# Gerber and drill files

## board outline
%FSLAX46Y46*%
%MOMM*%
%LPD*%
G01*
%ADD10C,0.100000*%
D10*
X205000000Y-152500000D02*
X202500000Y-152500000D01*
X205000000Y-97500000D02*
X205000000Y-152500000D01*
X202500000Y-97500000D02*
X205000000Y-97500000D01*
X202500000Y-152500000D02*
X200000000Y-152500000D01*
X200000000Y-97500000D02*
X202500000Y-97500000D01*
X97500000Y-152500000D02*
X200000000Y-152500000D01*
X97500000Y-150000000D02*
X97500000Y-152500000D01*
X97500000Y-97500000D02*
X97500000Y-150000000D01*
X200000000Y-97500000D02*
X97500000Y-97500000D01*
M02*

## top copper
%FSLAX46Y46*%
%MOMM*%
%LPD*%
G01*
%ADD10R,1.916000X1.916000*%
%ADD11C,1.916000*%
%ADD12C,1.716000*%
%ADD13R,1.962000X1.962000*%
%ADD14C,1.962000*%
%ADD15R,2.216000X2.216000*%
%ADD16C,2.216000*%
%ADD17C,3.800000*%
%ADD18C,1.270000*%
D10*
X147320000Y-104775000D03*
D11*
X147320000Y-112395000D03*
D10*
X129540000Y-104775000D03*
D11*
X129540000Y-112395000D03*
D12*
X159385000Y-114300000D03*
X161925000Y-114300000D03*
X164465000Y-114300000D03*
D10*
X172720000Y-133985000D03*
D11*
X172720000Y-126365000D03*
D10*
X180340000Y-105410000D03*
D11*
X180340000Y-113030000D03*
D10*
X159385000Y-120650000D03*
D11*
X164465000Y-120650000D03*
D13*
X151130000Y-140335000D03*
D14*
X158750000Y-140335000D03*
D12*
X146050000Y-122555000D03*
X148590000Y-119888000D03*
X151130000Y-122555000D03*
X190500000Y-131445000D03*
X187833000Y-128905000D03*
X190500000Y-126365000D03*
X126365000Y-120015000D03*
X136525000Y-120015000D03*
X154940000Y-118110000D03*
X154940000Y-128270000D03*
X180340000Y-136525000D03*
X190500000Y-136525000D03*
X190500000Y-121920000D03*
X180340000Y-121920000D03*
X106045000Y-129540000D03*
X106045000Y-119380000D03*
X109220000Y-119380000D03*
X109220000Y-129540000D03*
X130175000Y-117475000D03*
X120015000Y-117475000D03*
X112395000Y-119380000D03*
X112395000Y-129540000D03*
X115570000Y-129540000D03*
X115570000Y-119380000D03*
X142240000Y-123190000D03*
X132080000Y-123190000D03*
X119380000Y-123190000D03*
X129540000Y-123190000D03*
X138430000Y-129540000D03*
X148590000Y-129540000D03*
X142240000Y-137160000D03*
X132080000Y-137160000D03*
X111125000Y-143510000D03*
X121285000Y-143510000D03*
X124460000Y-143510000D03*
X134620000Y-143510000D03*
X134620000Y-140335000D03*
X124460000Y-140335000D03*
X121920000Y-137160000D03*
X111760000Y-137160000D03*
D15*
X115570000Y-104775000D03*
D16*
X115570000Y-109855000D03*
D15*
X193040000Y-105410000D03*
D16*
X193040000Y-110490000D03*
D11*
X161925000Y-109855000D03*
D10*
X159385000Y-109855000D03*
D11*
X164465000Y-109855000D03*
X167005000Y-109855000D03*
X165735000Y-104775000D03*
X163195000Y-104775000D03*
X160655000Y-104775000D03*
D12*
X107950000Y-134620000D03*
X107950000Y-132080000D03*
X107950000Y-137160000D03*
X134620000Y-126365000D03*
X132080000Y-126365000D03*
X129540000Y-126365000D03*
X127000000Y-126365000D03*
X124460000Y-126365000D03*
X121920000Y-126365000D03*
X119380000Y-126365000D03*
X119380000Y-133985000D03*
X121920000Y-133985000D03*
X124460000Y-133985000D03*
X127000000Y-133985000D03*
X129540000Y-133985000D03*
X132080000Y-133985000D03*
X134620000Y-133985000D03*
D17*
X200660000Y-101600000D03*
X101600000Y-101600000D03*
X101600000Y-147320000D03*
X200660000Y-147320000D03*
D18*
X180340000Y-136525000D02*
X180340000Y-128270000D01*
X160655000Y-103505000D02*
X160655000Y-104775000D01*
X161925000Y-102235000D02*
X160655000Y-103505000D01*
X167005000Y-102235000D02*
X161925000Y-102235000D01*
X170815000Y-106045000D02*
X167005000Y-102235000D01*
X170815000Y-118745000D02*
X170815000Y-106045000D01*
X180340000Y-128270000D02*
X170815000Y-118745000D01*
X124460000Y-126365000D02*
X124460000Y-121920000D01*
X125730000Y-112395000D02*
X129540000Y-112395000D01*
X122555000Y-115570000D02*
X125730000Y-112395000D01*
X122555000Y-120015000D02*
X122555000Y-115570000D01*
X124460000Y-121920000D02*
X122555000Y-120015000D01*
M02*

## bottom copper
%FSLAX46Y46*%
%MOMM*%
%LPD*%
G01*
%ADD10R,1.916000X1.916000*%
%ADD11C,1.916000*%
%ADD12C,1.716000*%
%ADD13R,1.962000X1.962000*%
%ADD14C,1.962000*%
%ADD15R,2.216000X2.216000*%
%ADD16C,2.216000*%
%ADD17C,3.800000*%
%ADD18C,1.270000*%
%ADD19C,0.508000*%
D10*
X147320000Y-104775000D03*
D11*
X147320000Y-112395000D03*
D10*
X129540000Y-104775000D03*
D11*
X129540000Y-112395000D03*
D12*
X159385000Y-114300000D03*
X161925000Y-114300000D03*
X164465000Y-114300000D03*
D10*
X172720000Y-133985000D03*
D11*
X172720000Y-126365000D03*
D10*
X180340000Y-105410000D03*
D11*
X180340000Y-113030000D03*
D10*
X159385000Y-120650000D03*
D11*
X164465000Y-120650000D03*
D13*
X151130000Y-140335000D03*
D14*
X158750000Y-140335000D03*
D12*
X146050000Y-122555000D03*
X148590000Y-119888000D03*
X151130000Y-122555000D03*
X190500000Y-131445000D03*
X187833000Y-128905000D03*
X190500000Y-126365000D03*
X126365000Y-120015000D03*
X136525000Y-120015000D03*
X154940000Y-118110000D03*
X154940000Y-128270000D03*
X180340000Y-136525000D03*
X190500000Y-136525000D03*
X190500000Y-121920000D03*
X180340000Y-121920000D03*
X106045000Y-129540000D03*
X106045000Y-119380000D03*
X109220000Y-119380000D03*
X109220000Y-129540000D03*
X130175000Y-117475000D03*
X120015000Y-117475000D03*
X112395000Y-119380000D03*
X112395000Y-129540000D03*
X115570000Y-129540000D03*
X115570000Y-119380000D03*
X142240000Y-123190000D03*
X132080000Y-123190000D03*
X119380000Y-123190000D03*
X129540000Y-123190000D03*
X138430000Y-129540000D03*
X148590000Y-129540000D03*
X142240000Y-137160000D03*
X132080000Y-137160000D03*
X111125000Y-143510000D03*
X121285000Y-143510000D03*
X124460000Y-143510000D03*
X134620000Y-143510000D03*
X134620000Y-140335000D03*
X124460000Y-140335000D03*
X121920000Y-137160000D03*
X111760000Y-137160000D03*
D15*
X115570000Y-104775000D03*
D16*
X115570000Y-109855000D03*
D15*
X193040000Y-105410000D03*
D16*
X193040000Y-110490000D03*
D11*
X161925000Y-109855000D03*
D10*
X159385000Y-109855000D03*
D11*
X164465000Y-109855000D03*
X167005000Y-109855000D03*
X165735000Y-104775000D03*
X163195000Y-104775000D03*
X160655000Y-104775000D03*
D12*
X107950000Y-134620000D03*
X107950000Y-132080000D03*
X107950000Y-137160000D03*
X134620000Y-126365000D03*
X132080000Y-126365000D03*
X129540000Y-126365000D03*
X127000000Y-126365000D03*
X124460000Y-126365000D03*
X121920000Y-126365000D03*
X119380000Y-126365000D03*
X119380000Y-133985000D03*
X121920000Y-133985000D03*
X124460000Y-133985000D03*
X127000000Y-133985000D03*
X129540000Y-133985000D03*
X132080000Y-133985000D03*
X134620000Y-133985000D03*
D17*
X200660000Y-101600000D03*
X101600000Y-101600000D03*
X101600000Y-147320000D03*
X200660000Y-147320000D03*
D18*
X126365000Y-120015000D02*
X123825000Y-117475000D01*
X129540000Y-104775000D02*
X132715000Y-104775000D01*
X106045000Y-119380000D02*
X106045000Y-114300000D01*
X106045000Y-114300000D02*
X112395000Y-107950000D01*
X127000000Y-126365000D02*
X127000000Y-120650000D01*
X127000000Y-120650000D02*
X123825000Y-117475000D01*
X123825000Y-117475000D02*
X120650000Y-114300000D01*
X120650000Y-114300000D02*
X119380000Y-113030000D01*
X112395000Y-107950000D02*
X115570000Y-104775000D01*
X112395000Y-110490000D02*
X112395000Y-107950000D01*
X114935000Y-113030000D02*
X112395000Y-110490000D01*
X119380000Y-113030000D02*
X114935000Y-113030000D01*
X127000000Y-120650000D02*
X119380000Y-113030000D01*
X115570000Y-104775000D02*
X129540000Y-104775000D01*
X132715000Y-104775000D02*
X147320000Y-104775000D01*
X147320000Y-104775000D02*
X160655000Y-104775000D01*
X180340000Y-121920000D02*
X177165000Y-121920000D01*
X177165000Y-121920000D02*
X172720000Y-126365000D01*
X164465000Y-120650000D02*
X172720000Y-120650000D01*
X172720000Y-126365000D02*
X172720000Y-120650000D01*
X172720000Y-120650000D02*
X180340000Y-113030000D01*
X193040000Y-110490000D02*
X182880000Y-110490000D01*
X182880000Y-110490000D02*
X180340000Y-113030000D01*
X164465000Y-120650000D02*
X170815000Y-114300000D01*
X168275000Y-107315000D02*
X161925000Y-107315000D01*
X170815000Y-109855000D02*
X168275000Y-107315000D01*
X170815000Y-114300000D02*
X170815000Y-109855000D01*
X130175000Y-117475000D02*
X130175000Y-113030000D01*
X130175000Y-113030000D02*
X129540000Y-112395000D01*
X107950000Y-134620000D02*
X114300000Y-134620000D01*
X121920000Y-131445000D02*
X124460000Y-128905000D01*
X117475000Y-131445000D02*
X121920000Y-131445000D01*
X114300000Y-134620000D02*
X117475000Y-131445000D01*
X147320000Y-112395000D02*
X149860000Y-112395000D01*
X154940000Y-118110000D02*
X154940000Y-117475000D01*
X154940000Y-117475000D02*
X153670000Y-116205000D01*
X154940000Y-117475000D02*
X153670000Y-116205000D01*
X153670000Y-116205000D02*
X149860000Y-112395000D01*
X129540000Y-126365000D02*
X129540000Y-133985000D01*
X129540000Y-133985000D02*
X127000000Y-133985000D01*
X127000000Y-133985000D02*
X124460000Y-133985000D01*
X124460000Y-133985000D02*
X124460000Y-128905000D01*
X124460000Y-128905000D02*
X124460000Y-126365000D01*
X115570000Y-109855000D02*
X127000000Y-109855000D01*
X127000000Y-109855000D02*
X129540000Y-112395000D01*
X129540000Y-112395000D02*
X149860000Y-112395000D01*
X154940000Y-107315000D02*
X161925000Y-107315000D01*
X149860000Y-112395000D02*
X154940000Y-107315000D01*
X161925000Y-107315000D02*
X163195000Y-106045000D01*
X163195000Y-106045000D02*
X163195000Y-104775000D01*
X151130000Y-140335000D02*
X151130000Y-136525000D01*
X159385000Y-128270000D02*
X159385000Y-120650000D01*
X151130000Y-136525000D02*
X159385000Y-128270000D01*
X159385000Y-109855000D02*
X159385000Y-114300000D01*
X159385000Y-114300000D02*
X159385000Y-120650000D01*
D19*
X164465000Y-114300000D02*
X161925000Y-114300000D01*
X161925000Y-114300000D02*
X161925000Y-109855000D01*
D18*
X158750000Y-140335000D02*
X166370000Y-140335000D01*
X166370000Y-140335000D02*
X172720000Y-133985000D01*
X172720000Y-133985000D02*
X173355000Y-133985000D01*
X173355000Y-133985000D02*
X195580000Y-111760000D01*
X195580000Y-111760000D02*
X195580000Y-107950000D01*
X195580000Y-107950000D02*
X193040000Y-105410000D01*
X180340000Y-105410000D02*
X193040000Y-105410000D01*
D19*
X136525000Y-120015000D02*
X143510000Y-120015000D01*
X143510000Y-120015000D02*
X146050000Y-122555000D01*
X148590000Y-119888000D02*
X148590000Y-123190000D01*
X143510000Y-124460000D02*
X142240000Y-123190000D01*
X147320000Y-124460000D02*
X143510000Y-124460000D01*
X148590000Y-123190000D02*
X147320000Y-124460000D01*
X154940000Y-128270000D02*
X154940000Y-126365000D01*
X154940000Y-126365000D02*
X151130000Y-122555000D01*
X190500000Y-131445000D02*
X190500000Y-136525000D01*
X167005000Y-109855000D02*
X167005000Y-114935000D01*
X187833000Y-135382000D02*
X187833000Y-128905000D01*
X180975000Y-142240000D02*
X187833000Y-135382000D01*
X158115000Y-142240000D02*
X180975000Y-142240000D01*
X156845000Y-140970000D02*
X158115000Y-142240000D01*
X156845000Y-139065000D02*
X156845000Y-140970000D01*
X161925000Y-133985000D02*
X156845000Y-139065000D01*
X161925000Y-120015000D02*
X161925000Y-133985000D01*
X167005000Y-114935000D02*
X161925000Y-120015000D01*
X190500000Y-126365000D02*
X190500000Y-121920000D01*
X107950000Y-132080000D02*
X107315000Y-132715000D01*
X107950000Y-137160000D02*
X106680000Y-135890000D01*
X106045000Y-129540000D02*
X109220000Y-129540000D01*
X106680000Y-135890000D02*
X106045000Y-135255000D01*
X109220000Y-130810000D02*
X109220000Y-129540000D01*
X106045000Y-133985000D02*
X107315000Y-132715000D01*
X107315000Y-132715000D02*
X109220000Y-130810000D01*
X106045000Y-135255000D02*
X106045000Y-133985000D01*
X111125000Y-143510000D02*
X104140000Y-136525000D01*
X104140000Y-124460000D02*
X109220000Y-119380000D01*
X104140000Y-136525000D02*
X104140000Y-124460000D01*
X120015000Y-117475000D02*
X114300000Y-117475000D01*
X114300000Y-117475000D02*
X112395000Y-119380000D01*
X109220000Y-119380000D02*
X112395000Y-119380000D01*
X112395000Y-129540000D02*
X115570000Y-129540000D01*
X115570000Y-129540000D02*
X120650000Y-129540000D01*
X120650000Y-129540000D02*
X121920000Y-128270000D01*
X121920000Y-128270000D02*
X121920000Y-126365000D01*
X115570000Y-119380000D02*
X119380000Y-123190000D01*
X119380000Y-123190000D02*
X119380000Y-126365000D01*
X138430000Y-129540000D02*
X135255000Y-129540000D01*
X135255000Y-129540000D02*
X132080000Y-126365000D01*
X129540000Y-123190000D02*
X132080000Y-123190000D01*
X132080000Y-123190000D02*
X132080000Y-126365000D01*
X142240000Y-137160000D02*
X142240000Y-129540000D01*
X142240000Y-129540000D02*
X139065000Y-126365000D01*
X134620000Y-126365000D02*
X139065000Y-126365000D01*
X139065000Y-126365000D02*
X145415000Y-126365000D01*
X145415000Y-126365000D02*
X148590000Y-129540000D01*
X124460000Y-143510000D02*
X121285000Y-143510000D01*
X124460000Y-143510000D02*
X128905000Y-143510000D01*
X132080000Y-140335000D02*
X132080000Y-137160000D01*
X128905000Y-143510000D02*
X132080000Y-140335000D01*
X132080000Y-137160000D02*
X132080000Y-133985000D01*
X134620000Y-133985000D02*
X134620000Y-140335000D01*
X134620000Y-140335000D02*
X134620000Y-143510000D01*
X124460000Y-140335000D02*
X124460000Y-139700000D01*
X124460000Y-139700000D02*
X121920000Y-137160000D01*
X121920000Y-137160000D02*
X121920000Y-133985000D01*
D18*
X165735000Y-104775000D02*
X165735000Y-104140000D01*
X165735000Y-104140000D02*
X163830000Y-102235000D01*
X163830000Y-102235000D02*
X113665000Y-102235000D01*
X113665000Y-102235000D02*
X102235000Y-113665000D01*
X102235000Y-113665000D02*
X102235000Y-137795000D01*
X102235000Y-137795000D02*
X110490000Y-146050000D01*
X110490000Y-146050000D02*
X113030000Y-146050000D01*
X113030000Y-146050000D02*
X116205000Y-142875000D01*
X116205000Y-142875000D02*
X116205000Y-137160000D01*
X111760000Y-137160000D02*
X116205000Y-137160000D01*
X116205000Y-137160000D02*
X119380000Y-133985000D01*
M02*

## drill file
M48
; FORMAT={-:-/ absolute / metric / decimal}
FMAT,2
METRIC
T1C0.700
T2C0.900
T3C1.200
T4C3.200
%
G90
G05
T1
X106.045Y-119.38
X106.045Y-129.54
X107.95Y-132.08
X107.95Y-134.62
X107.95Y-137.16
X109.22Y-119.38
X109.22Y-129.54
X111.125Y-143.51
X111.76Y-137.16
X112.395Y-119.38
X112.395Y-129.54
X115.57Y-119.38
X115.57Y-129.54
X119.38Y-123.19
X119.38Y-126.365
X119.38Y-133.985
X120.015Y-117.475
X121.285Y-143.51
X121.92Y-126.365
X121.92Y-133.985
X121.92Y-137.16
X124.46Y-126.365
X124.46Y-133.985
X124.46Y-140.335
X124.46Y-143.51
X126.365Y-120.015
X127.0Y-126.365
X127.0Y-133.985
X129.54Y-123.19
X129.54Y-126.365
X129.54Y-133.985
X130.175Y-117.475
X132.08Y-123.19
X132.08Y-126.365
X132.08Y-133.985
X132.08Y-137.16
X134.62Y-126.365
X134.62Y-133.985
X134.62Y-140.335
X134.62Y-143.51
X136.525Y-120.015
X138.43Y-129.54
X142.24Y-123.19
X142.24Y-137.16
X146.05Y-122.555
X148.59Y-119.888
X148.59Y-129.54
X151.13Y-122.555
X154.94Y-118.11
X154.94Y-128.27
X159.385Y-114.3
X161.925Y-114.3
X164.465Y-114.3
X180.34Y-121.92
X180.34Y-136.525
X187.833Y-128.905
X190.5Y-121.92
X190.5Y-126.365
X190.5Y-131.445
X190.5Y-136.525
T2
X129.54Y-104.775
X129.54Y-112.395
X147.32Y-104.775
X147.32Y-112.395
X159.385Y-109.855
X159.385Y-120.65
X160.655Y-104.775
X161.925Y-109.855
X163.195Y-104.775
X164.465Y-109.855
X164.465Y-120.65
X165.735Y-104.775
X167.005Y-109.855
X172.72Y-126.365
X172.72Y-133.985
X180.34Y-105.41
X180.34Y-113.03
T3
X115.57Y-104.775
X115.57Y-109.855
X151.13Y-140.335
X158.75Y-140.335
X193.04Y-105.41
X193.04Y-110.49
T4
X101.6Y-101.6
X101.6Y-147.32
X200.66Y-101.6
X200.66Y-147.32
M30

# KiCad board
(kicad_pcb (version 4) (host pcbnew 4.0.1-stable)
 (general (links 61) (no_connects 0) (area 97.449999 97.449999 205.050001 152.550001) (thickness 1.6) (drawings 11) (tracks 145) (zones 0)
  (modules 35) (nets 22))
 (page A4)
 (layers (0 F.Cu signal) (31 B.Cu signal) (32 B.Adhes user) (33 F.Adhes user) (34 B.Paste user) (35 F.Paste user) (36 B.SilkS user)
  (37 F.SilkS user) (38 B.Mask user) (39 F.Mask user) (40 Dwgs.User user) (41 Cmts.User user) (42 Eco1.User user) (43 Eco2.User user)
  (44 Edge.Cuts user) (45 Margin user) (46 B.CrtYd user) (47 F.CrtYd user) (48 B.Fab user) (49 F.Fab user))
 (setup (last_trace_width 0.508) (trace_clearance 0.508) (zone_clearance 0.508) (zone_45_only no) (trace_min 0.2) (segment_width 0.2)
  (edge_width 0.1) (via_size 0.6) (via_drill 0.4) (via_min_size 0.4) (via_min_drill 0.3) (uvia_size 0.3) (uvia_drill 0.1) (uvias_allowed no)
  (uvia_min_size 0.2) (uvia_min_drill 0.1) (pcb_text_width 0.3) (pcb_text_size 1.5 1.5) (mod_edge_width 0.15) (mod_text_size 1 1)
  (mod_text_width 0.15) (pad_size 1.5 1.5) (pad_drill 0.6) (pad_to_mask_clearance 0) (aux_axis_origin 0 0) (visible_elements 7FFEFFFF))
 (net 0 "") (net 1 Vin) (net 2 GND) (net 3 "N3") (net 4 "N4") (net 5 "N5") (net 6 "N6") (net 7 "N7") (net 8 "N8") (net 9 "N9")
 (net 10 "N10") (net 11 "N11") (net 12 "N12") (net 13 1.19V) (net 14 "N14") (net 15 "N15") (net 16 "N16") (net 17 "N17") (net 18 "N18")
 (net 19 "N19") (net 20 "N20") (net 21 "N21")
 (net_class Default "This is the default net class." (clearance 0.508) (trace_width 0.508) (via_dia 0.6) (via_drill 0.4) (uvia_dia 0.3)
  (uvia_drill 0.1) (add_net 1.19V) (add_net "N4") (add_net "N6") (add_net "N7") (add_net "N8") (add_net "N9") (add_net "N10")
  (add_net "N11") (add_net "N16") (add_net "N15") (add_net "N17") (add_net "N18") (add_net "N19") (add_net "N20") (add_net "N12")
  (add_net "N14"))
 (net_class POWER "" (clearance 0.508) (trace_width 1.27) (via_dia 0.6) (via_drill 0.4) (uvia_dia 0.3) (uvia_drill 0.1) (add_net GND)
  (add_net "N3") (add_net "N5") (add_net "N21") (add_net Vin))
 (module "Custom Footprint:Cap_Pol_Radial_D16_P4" (layer F.Cu) (at 147.32 108.585 270)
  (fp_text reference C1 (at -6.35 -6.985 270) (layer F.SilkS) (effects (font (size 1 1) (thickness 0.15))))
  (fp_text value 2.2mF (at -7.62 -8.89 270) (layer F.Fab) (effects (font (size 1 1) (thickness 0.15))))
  (pad 1 thru_hole rect (at -3.81 0 270) (size 1.916 1.916) (drill 0.9) (layers *.Cu *.Mask F.SilkS) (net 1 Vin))
  (pad 2 thru_hole circle (at 3.81 0 270) (size 1.916 1.916) (drill 0.9) (layers *.Cu *.Mask F.SilkS) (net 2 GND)))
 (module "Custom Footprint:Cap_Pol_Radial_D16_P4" (layer F.Cu) (at 129.54 108.585 270)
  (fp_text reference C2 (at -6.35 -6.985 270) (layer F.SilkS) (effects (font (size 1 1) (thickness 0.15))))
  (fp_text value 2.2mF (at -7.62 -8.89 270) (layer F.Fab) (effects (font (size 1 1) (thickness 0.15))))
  (pad 1 thru_hole rect (at -3.81 0 270) (size 1.916 1.916) (drill 0.9) (layers *.Cu *.Mask F.SilkS) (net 1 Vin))
  (pad 2 thru_hole circle (at 3.81 0 270) (size 1.916 1.916) (drill 0.9) (layers *.Cu *.Mask F.SilkS) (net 2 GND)))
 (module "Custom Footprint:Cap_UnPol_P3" (layer F.Cu) (at 159.385 114.3 90)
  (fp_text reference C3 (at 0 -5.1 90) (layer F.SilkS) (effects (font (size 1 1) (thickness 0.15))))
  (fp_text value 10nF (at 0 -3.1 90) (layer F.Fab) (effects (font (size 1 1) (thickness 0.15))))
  (pad 1 thru_hole circle (at 0 0 90) (size 1.716 1.716) (drill 0.7) (layers *.Cu *.Mask F.SilkS) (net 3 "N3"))
  (pad 2 thru_hole circle (at 0 2.54 90) (size 1.716 1.716) (drill 0.7) (layers *.Cu *.Mask F.SilkS) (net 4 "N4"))
  (pad 2 thru_hole circle (at 0 5.08 90) (size 1.716 1.716) (drill 0.7) (layers *.Cu *.Mask F.SilkS) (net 4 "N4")))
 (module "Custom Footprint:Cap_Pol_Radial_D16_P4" (layer F.Cu) (at 172.72 130.175 90)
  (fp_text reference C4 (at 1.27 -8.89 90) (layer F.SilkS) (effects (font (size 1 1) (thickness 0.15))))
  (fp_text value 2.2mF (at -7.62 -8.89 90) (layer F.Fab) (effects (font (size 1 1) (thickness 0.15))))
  (pad 1 thru_hole rect (at -3.81 0 90) (size 1.916 1.916) (drill 0.9) (layers *.Cu *.Mask F.SilkS) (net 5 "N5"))
  (pad 2 thru_hole circle (at 3.81 0 90) (size 1.916 1.916) (drill 0.9) (layers *.Cu *.Mask F.SilkS) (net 2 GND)))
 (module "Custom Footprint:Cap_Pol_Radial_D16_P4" (layer F.Cu) (at 180.34 109.22 270)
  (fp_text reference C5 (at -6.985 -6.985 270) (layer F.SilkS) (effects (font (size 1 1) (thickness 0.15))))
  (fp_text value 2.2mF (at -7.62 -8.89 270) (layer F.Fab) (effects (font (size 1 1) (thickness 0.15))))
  (pad 1 thru_hole rect (at -3.81 0 270) (size 1.916 1.916) (drill 0.9) (layers *.Cu *.Mask F.SilkS) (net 5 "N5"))
  (pad 2 thru_hole circle (at 3.81 0 270) (size 1.916 1.916) (drill 0.9) (layers *.Cu *.Mask F.SilkS) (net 2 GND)))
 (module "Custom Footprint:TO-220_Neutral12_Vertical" (layer F.Cu) (at 161.925 120.65)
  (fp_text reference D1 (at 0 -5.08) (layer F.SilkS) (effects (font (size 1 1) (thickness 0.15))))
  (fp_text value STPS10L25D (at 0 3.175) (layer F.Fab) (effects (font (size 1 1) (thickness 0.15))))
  (pad 1 thru_hole rect (at -2.54 0 90) (size 1.916 1.916) (drill 0.9) (layers *.Cu *.Mask F.SilkS) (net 3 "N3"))
  (pad 2 thru_hole circle (at 2.54 0 90) (size 1.916 1.916) (drill 0.9) (layers *.Cu *.Mask F.SilkS) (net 2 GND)))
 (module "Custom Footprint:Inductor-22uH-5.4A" (layer F.Cu) (at 154.94 140.335)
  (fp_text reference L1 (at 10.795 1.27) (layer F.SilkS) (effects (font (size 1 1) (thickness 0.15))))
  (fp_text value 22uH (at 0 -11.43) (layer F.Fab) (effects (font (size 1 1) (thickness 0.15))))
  (pad 1 thru_hole rect (at -3.81 0) (size 1.962 1.962) (drill 1.2) (layers *.Cu *.Mask F.SilkS) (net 3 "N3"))
  (pad 2 thru_hole circle (at 3.81 0) (size 1.962 1.962) (drill 1.2) (layers *.Cu *.Mask F.SilkS) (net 5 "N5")))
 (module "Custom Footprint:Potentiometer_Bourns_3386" (layer F.Cu) (at 146.05 122.555 180)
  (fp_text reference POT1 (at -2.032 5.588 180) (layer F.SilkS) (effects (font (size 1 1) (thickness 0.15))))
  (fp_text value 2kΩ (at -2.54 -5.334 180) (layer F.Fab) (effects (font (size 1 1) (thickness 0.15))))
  (pad 1 thru_hole circle (at 0 0 180) (size 1.716 1.716) (drill 0.7) (layers *.Cu *.Mask F.SilkS) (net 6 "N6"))
  (pad 2 thru_hole circle (at -2.54 2.667 180) (size 1.716 1.716) (drill 0.7) (layers *.Cu *.Mask F.SilkS) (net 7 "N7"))
  (pad 3 thru_hole circle (at -5.08 0 180) (size 1.716 1.716) (drill 0.7) (layers *.Cu *.Mask F.SilkS) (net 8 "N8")))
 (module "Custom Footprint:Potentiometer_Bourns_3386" (layer F.Cu) (at 190.5 131.445 270)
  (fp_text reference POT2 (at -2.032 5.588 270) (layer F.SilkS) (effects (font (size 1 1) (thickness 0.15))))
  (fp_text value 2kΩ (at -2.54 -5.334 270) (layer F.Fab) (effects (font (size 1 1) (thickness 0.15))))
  (pad 1 thru_hole circle (at 0 0 270) (size 1.716 1.716) (drill 0.7) (layers *.Cu *.Mask F.SilkS) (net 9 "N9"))
  (pad 2 thru_hole circle (at -2.54 2.667 270) (size 1.716 1.716) (drill 0.7) (layers *.Cu *.Mask F.SilkS) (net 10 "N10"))
  (pad 3 thru_hole circle (at -5.08 0 270) (size 1.716 1.716) (drill 0.7) (layers *.Cu *.Mask F.SilkS) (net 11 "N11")))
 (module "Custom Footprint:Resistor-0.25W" (layer F.Cu) (at 126.365 120.015)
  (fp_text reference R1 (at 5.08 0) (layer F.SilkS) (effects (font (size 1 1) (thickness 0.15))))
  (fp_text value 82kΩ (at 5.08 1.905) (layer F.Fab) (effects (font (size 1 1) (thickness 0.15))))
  (pad 1 thru_hole circle (at 0 0) (size 1.716 1.716) (drill 0.7) (layers *.Cu *.Mask F.SilkS) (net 1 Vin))
  (pad 2 thru_hole circle (at 10.16 0) (size 1.716 1.716) (drill 0.7) (layers *.Cu *.Mask F.SilkS) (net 6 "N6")))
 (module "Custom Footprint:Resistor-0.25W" (layer F.Cu) (at 154.94 118.11 270)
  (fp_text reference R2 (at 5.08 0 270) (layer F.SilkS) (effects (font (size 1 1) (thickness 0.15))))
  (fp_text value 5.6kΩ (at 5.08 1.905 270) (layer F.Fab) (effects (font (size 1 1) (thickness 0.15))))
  (pad 1 thru_hole circle (at 0 0 270) (size 1.716 1.716) (drill 0.7) (layers *.Cu *.Mask F.SilkS) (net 2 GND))
  (pad 2 thru_hole circle (at 10.16 0 270) (size 1.716 1.716) (drill 0.7) (layers *.Cu *.Mask F.SilkS) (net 8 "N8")))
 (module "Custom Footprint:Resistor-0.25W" (layer F.Cu) (at 180.34 136.525)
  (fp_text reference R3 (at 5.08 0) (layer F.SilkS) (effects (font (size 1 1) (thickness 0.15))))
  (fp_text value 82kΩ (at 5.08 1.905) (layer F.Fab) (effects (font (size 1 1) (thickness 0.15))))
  (pad 1 thru_hole circle (at 0 0) (size 1.716 1.716) (drill 0.7) (layers *.Cu *.Mask F.SilkS) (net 1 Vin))
  (pad 2 thru_hole circle (at 10.16 0) (size 1.716 1.716) (drill 0.7) (layers *.Cu *.Mask F.SilkS) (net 9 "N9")))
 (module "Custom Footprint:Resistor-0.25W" (layer F.Cu) (at 190.5 121.92 180)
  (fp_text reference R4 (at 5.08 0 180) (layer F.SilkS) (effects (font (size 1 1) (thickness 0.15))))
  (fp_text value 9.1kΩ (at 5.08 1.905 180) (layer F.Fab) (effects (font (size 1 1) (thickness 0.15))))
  (pad 1 thru_hole circle (at 0 0 180) (size 1.716 1.716) (drill 0.7) (layers *.Cu *.Mask F.SilkS) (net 11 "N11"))
  (pad 2 thru_hole circle (at 10.16 0 180) (size 1.716 1.716) (drill 0.7) (layers *.Cu *.Mask F.SilkS) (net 2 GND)))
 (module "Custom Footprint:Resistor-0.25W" (layer F.Cu) (at 106.045 129.54 90)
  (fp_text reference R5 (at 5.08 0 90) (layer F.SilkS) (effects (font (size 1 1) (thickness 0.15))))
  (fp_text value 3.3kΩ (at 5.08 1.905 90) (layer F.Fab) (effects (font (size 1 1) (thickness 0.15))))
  (pad 1 thru_hole circle (at 0 0 90) (size 1.716 1.716) (drill 0.7) (layers *.Cu *.Mask F.SilkS) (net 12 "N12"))
  (pad 2 thru_hole circle (at 10.16 0 90) (size 1.716 1.716) (drill 0.7) (layers *.Cu *.Mask F.SilkS) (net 1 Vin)))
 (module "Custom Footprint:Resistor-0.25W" (layer F.Cu) (at 109.22 119.38 270)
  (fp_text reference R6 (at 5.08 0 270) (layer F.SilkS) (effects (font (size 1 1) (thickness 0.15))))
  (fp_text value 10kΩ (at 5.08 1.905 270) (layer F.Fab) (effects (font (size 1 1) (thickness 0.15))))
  (pad 1 thru_hole circle (at 0 0 270) (size 1.716 1.716) (drill 0.7) (layers *.Cu *.Mask F.SilkS) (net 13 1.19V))
  (pad 2 thru_hole circle (at 10.16 0 270) (size 1.716 1.716) (drill 0.7) (layers *.Cu *.Mask F.SilkS) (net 12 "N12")))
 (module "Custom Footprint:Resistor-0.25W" (layer F.Cu) (at 130.175 117.475 180)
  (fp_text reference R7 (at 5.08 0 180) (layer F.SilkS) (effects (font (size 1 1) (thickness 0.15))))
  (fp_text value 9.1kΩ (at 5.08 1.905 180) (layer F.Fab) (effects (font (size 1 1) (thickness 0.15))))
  (pad 1 thru_hole circle (at 0 0 180) (size 1.716 1.716) (drill 0.7) (layers *.Cu *.Mask F.SilkS) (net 2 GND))
  (pad 2 thru_hole circle (at 10.16 0 180) (size 1.716 1.716) (drill 0.7) (layers *.Cu *.Mask F.SilkS) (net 13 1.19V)))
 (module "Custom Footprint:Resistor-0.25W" (layer F.Cu) (at 112.395 119.38 270)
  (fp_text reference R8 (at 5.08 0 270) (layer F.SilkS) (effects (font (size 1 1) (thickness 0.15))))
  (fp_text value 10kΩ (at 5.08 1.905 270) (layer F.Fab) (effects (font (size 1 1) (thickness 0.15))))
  (pad 1 thru_hole circle (at 0 0 270) (size 1.716 1.716) (drill 0.7) (layers *.Cu *.Mask F.SilkS) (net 13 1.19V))
  (pad 2 thru_hole circle (at 10.16 0 270) (size 1.716 1.716) (drill 0.7) (layers *.Cu *.Mask F.SilkS) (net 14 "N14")))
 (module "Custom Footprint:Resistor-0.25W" (layer F.Cu) (at 115.57 129.54 90)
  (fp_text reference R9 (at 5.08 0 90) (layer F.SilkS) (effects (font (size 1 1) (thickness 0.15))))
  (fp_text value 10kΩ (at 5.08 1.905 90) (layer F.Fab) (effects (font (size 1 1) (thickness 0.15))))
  (pad 1 thru_hole circle (at 0 0 90) (size 1.716 1.716) (drill 0.7) (layers *.Cu *.Mask F.SilkS) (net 14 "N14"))
  (pad 2 thru_hole circle (at 10.16 0 90) (size 1.716 1.716) (drill 0.7) (layers *.Cu *.Mask F.SilkS) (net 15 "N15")))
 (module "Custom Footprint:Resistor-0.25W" (layer F.Cu) (at 142.24 123.19 180)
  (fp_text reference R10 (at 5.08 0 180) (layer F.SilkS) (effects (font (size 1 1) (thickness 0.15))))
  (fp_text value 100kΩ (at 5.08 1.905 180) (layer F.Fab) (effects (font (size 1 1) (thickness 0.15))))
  (pad 1 thru_hole circle (at 0 0 180) (size 1.716 1.716) (drill 0.7) (layers *.Cu *.Mask F.SilkS) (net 7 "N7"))
  (pad 2 thru_hole circle (at 10.16 0 180) (size 1.716 1.716) (drill 0.7) (layers *.Cu *.Mask F.SilkS) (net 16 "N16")))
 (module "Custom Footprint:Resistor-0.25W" (layer F.Cu) (at 119.38 123.19)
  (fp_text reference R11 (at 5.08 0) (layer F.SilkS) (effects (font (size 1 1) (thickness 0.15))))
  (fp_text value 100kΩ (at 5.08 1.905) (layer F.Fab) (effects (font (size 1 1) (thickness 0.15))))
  (pad 1 thru_hole circle (at 0 0) (size 1.716 1.716) (drill 0.7) (layers *.Cu *.Mask F.SilkS) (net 15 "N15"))
  (pad 2 thru_hole circle (at 10.16 0) (size 1.716 1.716) (drill 0.7) (layers *.Cu *.Mask F.SilkS) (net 16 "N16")))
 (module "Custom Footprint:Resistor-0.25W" (layer F.Cu) (at 138.43 129.54)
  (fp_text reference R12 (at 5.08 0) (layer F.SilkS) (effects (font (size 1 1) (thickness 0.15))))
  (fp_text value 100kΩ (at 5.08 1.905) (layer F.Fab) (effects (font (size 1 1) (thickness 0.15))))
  (pad 1 thru_hole circle (at 0 0) (size 1.716 1.716) (drill 0.7) (layers *.Cu *.Mask F.SilkS) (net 16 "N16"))
  (pad 2 thru_hole circle (at 10.16 0) (size 1.716 1.716) (drill 0.7) (layers *.Cu *.Mask F.SilkS) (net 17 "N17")))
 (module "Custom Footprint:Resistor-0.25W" (layer F.Cu) (at 142.24 137.16 180)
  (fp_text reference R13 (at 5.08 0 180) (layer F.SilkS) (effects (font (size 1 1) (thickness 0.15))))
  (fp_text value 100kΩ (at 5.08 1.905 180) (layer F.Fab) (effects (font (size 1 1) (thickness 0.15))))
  (pad 1 thru_hole circle (at 0 0 180) (size 1.716 1.716) (drill 0.7) (layers *.Cu *.Mask F.SilkS) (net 17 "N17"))
  (pad 2 thru_hole circle (at 10.16 0 180) (size 1.716 1.716) (drill 0.7) (layers *.Cu *.Mask F.SilkS) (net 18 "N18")))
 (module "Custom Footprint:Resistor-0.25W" (layer F.Cu) (at 111.125 143.51)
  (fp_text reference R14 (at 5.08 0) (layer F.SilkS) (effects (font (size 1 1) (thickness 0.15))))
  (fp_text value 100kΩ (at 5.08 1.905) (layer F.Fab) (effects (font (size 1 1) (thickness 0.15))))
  (pad 1 thru_hole circle (at 0 0) (size 1.716 1.716) (drill 0.7) (layers *.Cu *.Mask F.SilkS) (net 13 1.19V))
  (pad 2 thru_hole circle (at 10.16 0) (size 1.716 1.716) (drill 0.7) (layers *.Cu *.Mask F.SilkS) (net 18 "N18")))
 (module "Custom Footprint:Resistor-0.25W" (layer F.Cu) (at 124.46 143.51)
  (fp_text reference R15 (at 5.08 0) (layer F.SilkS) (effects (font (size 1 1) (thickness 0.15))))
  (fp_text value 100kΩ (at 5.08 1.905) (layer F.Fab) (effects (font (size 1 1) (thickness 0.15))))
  (pad 1 thru_hole circle (at 0 0) (size 1.716 1.716) (drill 0.7) (layers *.Cu *.Mask F.SilkS) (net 18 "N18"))
  (pad 2 thru_hole circle (at 10.16 0) (size 1.716 1.716) (drill 0.7) (layers *.Cu *.Mask F.SilkS) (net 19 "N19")))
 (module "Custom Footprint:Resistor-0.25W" (layer F.Cu) (at 134.62 140.335 180)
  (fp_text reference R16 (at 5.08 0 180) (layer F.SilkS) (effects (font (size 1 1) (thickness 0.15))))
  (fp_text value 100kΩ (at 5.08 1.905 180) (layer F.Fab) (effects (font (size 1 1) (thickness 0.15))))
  (pad 1 thru_hole circle (at 0 0 180) (size 1.716 1.716) (drill 0.7) (layers *.Cu *.Mask F.SilkS) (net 19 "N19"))
  (pad 2 thru_hole circle (at 10.16 0 180) (size 1.716 1.716) (drill 0.7) (layers *.Cu *.Mask F.SilkS) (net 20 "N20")))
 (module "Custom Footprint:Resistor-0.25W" (layer F.Cu) (at 121.92 137.16 180)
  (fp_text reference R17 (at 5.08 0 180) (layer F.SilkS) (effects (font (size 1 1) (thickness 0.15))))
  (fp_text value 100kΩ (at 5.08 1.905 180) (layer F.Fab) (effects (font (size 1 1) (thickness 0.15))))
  (pad 1 thru_hole circle (at 0 0 180) (size 1.716 1.716) (drill 0.7) (layers *.Cu *.Mask F.SilkS) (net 20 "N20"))
  (pad 2 thru_hole circle (at 10.16 0 180) (size 1.716 1.716) (drill 0.7) (layers *.Cu *.Mask F.SilkS) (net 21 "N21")))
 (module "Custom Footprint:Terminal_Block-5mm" (layer F.Cu) (at 115.57 107.315 270)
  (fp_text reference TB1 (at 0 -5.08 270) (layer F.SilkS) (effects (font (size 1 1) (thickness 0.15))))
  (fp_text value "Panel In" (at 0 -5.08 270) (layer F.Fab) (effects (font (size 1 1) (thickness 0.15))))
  (pad 1 thru_hole rect (at -2.54 0 270) (size 2.216 2.216) (drill 1.2) (layers *.Cu *.Mask F.SilkS) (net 1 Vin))
  (pad 2 thru_hole circle (at 2.54 0 270) (size 2.216 2.216) (drill 1.2) (layers *.Cu *.Mask F.SilkS) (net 2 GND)))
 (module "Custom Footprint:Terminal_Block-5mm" (layer F.Cu) (at 193.04 107.95 270)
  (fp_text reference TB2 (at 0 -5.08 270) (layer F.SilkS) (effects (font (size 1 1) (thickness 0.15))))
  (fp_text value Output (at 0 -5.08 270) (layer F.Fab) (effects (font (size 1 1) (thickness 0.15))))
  (pad 1 thru_hole rect (at -2.54 0 270) (size 2.216 2.216) (drill 1.2) (layers *.Cu *.Mask F.SilkS) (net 5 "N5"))
  (pad 2 thru_hole circle (at 2.54 0 270) (size 2.216 2.216) (drill 1.2) (layers *.Cu *.Mask F.SilkS) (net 2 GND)))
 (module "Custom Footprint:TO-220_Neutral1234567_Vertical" (layer F.Cu) (at 164.465 109.855 180)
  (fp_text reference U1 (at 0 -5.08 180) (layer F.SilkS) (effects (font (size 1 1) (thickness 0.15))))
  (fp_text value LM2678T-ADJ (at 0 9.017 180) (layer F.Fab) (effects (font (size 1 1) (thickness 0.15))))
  (pad 3 thru_hole circle (at 2.54 0 270) (size 1.916 1.916) (drill 0.9) (layers *.Cu *.Mask F.SilkS) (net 4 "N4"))
  (pad 1 thru_hole rect (at 5.08 0 270) (size 1.916 1.916) (drill 0.9) (layers *.Cu *.Mask F.SilkS) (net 3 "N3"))
  (pad 5 thru_hole circle (at 0 0 270) (size 1.916 1.916) (drill 0.9) (layers *.Cu *.Mask F.SilkS))
  (pad 7 thru_hole circle (at -2.54 0 270) (size 1.916 1.916) (drill 0.9) (layers *.Cu *.Mask F.SilkS) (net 10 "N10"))
  (pad 6 thru_hole circle (at -1.27 5.08 270) (size 1.916 1.916) (drill 0.9) (layers *.Cu *.Mask F.SilkS) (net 21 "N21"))
  (pad 4 thru_hole circle (at 1.27 5.08 270) (size 1.916 1.916) (drill 0.9) (layers *.Cu *.Mask F.SilkS) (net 2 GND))
  (pad 2 thru_hole circle (at 3.81 5.08 270) (size 1.916 1.916) (drill 0.9) (layers *.Cu *.Mask F.SilkS) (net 1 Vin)))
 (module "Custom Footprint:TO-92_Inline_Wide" (layer F.Cu) (at 107.95 137.16 90)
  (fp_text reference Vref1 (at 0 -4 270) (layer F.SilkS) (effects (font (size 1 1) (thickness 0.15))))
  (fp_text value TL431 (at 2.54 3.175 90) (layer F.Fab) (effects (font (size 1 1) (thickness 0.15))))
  (pad 2 thru_hole circle (at 2.54 0 180) (size 1.716 1.716) (drill 0.7) (layers *.Cu *.Mask F.SilkS) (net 2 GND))
  (pad 3 thru_hole circle (at 5.08 0 180) (size 1.716 1.716) (drill 0.7) (layers *.Cu *.Mask F.SilkS) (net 12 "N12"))
  (pad 1 thru_hole circle (at 0 0 180) (size 1.716 1.716) (drill 0.7) (layers *.Cu *.Mask F.SilkS) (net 12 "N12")))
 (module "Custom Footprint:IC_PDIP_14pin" (layer F.Cu) (at 134.62 126.365 270)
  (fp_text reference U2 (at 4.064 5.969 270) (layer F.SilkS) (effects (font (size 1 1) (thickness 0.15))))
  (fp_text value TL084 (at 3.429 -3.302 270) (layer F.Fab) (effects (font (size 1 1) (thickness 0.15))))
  (pad 1 thru_hole circle (at 0 0 270) (size 1.716 1.716) (drill 0.7) (layers *.Cu *.Mask F.SilkS) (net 17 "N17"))
  (pad 2 thru_hole circle (at 0 2.54 270) (size 1.716 1.716) (drill 0.7) (layers *.Cu *.Mask F.SilkS) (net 16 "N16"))
  (pad 3 thru_hole circle (at 0 5.08 270) (size 1.716 1.716) (drill 0.7) (layers *.Cu *.Mask F.SilkS) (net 2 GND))
  (pad 4 thru_hole circle (at 0 7.62 270) (size 1.716 1.716) (drill 0.7) (layers *.Cu *.Mask F.SilkS) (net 1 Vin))
  (pad 5 thru_hole circle (at 0 10.16 270) (size 1.716 1.716) (drill 0.7) (layers *.Cu *.Mask F.SilkS) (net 2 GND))
  (pad 6 thru_hole circle (at 0 12.7 270) (size 1.716 1.716) (drill 0.7) (layers *.Cu *.Mask F.SilkS) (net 14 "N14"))
  (pad 7 thru_hole circle (at 0 15.24 270) (size 1.716 1.716) (drill 0.7) (layers *.Cu *.Mask F.SilkS) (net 15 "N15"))
  (pad 8 thru_hole circle (at 7.62 15.24 270) (size 1.716 1.716) (drill 0.7) (layers *.Cu *.Mask F.SilkS) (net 21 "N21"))
  (pad 9 thru_hole circle (at 7.62 12.7 270) (size 1.716 1.716) (drill 0.7) (layers *.Cu *.Mask F.SilkS) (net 20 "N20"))
  (pad 10 thru_hole circle (at 7.62 10.16 270) (size 1.716 1.716) (drill 0.7) (layers *.Cu *.Mask F.SilkS) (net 2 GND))
  (pad 11 thru_hole circle (at 7.62 7.62 270) (size 1.716 1.716) (drill 0.7) (layers *.Cu *.Mask F.SilkS) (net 2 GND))
  (pad 12 thru_hole circle (at 7.62 5.08 270) (size 1.716 1.716) (drill 0.7) (layers *.Cu *.Mask F.SilkS) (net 2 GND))
  (pad 13 thru_hole circle (at 7.62 2.54 270) (size 1.716 1.716) (drill 0.7) (layers *.Cu *.Mask F.SilkS) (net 18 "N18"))
  (pad 14 thru_hole circle (at 7.62 0 270) (size 1.716 1.716) (drill 0.7) (layers *.Cu *.Mask F.SilkS) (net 19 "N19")))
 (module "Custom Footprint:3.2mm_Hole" (layer F.Cu) (at 200.66 101.6)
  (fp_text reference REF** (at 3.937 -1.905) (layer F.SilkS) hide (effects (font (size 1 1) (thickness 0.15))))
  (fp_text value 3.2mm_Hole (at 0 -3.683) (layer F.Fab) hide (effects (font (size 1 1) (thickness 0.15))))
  (pad 1 thru_hole circle (at 0 0) (size 3.8 3.8) (drill 3.2) (layers *.Cu *.Mask F.SilkS)))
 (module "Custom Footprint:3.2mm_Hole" (layer F.Cu) (at 101.6 101.6)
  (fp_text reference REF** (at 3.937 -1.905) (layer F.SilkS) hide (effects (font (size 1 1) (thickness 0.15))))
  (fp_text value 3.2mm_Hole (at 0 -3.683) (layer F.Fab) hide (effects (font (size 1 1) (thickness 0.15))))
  (pad 1 thru_hole circle (at 0 0) (size 3.8 3.8) (drill 3.2) (layers *.Cu *.Mask F.SilkS)))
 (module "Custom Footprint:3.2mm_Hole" (layer F.Cu) (at 101.6 147.32)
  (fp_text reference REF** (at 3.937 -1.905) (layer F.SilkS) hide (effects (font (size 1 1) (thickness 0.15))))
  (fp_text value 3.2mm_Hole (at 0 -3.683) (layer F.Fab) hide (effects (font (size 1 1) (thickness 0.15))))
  (pad 1 thru_hole circle (at 0 0) (size 3.8 3.8) (drill 3.2) (layers *.Cu *.Mask F.SilkS)))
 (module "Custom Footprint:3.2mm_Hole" (layer F.Cu) (at 200.66 147.32)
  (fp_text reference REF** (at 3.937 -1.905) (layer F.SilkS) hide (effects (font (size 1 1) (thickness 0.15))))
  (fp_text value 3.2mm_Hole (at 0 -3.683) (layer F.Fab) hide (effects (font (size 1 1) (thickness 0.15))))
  (pad 1 thru_hole circle (at 0 0) (size 3.8 3.8) (drill 3.2) (layers *.Cu *.Mask F.SilkS)))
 (gr_line (start 205 152.5) (end 202.5 152.5) (angle 90) (layer Edge.Cuts) (width 0.1))
 (gr_line (start 205 97.5) (end 205 152.5) (angle 90) (layer Edge.Cuts) (width 0.1))
 (gr_line (start 202.5 97.5) (end 205 97.5) (angle 90) (layer Edge.Cuts) (width 0.1))
 (gr_line (start 202.5 152.5) (end 200 152.5) (angle 90) (layer Edge.Cuts) (width 0.1))
 (gr_line (start 200 97.5) (end 202.5 97.5) (angle 90) (layer Edge.Cuts) (width 0.1))
 (gr_line (start 97.5 152.5) (end 200 152.5) (angle 90) (layer Edge.Cuts) (width 0.1))
 (gr_line (start 97.5 150) (end 97.5 152.5) (angle 90) (layer Edge.Cuts) (width 0.1))
 (gr_line (start 97.5 97.5) (end 97.5 150) (angle 90) (layer Edge.Cuts) (width 0.1))
 (gr_line (start 200 97.5) (end 97.5 97.5) (angle 90) (layer Edge.Cuts) (width 0.1))
 (segment (start 180.34 136.525) (end 180.34 128.27) (width 1.27) (layer F.Cu) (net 1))
 (segment (start 160.655 103.505) (end 160.655 104.775) (width 1.27) (layer F.Cu) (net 1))
 (segment (start 161.925 102.235) (end 160.655 103.505) (width 1.27) (layer F.Cu) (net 1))
 (segment (start 167.005 102.235) (end 161.925 102.235) (width 1.27) (layer F.Cu) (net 1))
 (segment (start 170.815 106.045) (end 167.005 102.235) (width 1.27) (layer F.Cu) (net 1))
 (segment (start 170.815 118.745) (end 170.815 106.045) (width 1.27) (layer F.Cu) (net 1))
 (segment (start 180.34 128.27) (end 170.815 118.745) (width 1.27) (layer F.Cu) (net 1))
 (segment (start 126.365 120.015) (end 123.825 117.475) (width 1.27) (layer B.Cu) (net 1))
 (segment (start 129.54 104.775) (end 132.715 104.775) (width 1.27) (layer B.Cu) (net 1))
 (segment (start 106.045 119.38) (end 106.045 114.3) (width 1.27) (layer B.Cu) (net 1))
 (segment (start 106.045 114.3) (end 112.395 107.95) (width 1.27) (layer B.Cu) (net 1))
 (segment (start 127 126.365) (end 127 120.65) (width 1.27) (layer B.Cu) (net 1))
 (segment (start 127 120.65) (end 123.825 117.475) (width 1.27) (layer B.Cu) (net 1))
 (segment (start 123.825 117.475) (end 120.65 114.3) (width 1.27) (layer B.Cu) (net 1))
 (segment (start 120.65 114.3) (end 119.38 113.03) (width 1.27) (layer B.Cu) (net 1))
 (segment (start 112.395 107.95) (end 115.57 104.775) (width 1.27) (layer B.Cu) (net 1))
 (segment (start 112.395 110.49) (end 112.395 107.95) (width 1.27) (layer B.Cu) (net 1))
 (segment (start 114.935 113.03) (end 112.395 110.49) (width 1.27) (layer B.Cu) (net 1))
 (segment (start 119.38 113.03) (end 114.935 113.03) (width 1.27) (layer B.Cu) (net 1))
 (segment (start 127 120.65) (end 119.38 113.03) (width 1.27) (layer B.Cu) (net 1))
 (segment (start 115.57 104.775) (end 129.54 104.775) (width 1.27) (layer B.Cu) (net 1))
 (segment (start 132.715 104.775) (end 147.32 104.775) (width 1.27) (layer B.Cu) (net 1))
 (segment (start 147.32 104.775) (end 160.655 104.775) (width 1.27) (layer B.Cu) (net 1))
 (segment (start 124.46 126.365) (end 124.46 121.92) (width 1.27) (layer F.Cu) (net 2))
 (segment (start 125.73 112.395) (end 129.54 112.395) (width 1.27) (layer F.Cu) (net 2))
 (segment (start 122.555 115.57) (end 125.73 112.395) (width 1.27) (layer F.Cu) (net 2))
 (segment (start 122.555 120.015) (end 122.555 115.57) (width 1.27) (layer F.Cu) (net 2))
 (segment (start 124.46 121.92) (end 122.555 120.015) (width 1.27) (layer F.Cu) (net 2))
 (segment (start 180.34 121.92) (end 177.165 121.92) (width 1.27) (layer B.Cu) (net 2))
 (segment (start 177.165 121.92) (end 172.72 126.365) (width 1.27) (layer B.Cu) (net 2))
 (segment (start 164.465 120.65) (end 172.72 120.65) (width 1.27) (layer B.Cu) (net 2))
 (segment (start 172.72 126.365) (end 172.72 120.65) (width 1.27) (layer B.Cu) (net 2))
 (segment (start 172.72 120.65) (end 180.34 113.03) (width 1.27) (layer B.Cu) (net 2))
 (segment (start 193.04 110.49) (end 182.88 110.49) (width 1.27) (layer B.Cu) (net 2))
 (segment (start 182.88 110.49) (end 180.34 113.03) (width 1.27) (layer B.Cu) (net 2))
 (segment (start 164.465 120.65) (end 170.815 114.3) (width 1.27) (layer B.Cu) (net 2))
 (segment (start 168.275 107.315) (end 161.925 107.315) (width 1.27) (layer B.Cu) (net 2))
 (segment (start 170.815 109.855) (end 168.275 107.315) (width 1.27) (layer B.Cu) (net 2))
 (segment (start 170.815 114.3) (end 170.815 109.855) (width 1.27) (layer B.Cu) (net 2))
 (segment (start 130.175 117.475) (end 130.175 113.03) (width 1.27) (layer B.Cu) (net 2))
 (segment (start 130.175 113.03) (end 129.54 112.395) (width 1.27) (layer B.Cu) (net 2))
 (segment (start 107.95 134.62) (end 114.3 134.62) (width 1.27) (layer B.Cu) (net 2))
 (segment (start 121.92 131.445) (end 124.46 128.905) (width 1.27) (layer B.Cu) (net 2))
 (segment (start 117.475 131.445) (end 121.92 131.445) (width 1.27) (layer B.Cu) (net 2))
 (segment (start 114.3 134.62) (end 117.475 131.445) (width 1.27) (layer B.Cu) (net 2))
 (segment (start 147.32 112.395) (end 149.86 112.395) (width 1.27) (layer B.Cu) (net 2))
 (segment (start 154.94 118.11) (end 154.94 117.475) (width 1.27) (layer B.Cu) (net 2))
 (segment (start 154.94 117.475) (end 153.67 116.205) (width 1.27) (layer B.Cu) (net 2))
 (segment (start 154.94 117.475) (end 153.67 116.205) (width 1.27) (layer B.Cu) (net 2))
 (segment (start 153.67 116.205) (end 149.86 112.395) (width 1.27) (layer B.Cu) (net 2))
 (segment (start 129.54 126.365) (end 129.54 133.985) (width 1.27) (layer B.Cu) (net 2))
 (segment (start 129.54 133.985) (end 127 133.985) (width 1.27) (layer B.Cu) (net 2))
 (segment (start 127 133.985) (end 124.46 133.985) (width 1.27) (layer B.Cu) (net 2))
 (segment (start 124.46 133.985) (end 124.46 128.905) (width 1.27) (layer B.Cu) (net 2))
 (segment (start 124.46 128.905) (end 124.46 126.365) (width 1.27) (layer B.Cu) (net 2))
 (segment (start 115.57 109.855) (end 127 109.855) (width 1.27) (layer B.Cu) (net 2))
 (segment (start 127 109.855) (end 129.54 112.395) (width 1.27) (layer B.Cu) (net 2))
 (segment (start 129.54 112.395) (end 149.86 112.395) (width 1.27) (layer B.Cu) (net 2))
 (segment (start 154.94 107.315) (end 161.925 107.315) (width 1.27) (layer B.Cu) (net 2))
 (segment (start 149.86 112.395) (end 154.94 107.315) (width 1.27) (layer B.Cu) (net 2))
 (segment (start 161.925 107.315) (end 163.195 106.045) (width 1.27) (layer B.Cu) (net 2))
 (segment (start 163.195 106.045) (end 163.195 104.775) (width 1.27) (layer B.Cu) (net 2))
 (segment (start 151.13 140.335) (end 151.13 136.525) (width 1.27) (layer B.Cu) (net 3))
 (segment (start 159.385 128.27) (end 159.385 120.65) (width 1.27) (layer B.Cu) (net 3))
 (segment (start 151.13 136.525) (end 159.385 128.27) (width 1.27) (layer B.Cu) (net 3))
 (segment (start 159.385 109.855) (end 159.385 114.3) (width 1.27) (layer B.Cu) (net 3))
 (segment (start 159.385 114.3) (end 159.385 120.65) (width 1.27) (layer B.Cu) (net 3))
 (segment (start 164.465 114.3) (end 161.925 114.3) (width 0.508) (layer B.Cu) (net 4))
 (segment (start 161.925 114.3) (end 161.925 109.855) (width 0.508) (layer B.Cu) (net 4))
 (segment (start 158.75 140.335) (end 166.37 140.335) (width 1.27) (layer B.Cu) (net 5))
 (segment (start 166.37 140.335) (end 172.72 133.985) (width 1.27) (layer B.Cu) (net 5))
 (segment (start 172.72 133.985) (end 173.355 133.985) (width 1.27) (layer B.Cu) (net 5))
 (segment (start 173.355 133.985) (end 195.58 111.76) (width 1.27) (layer B.Cu) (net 5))
 (segment (start 195.58 111.76) (end 195.58 107.95) (width 1.27) (layer B.Cu) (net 5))
 (segment (start 195.58 107.95) (end 193.04 105.41) (width 1.27) (layer B.Cu) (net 5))
 (segment (start 180.34 105.41) (end 193.04 105.41) (width 1.27) (layer B.Cu) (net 5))
 (segment (start 136.525 120.015) (end 143.51 120.015) (width 0.508) (layer B.Cu) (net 6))
 (segment (start 143.51 120.015) (end 146.05 122.555) (width 0.508) (layer B.Cu) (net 6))
 (segment (start 148.59 119.888) (end 148.59 123.19) (width 0.508) (layer B.Cu) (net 7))
 (segment (start 143.51 124.46) (end 142.24 123.19) (width 0.508) (layer B.Cu) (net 7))
 (segment (start 147.32 124.46) (end 143.51 124.46) (width 0.508) (layer B.Cu) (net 7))
 (segment (start 148.59 123.19) (end 147.32 124.46) (width 0.508) (layer B.Cu) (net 7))
 (segment (start 154.94 128.27) (end 154.94 126.365) (width 0.508) (layer B.Cu) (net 8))
 (segment (start 154.94 126.365) (end 151.13 122.555) (width 0.508) (layer B.Cu) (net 8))
 (segment (start 190.5 131.445) (end 190.5 136.525) (width 0.508) (layer B.Cu) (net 9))
 (segment (start 167.005 109.855) (end 167.005 114.935) (width 0.508) (layer B.Cu) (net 10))
 (segment (start 187.833 135.382) (end 187.833 128.905) (width 0.508) (layer B.Cu) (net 10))
 (segment (start 180.975 142.24) (end 187.833 135.382) (width 0.508) (layer B.Cu) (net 10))
 (segment (start 158.115 142.24) (end 180.975 142.24) (width 0.508) (layer B.Cu) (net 10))
 (segment (start 156.845 140.97) (end 158.115 142.24) (width 0.508) (layer B.Cu) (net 10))
 (segment (start 156.845 139.065) (end 156.845 140.97) (width 0.508) (layer B.Cu) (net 10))
 (segment (start 161.925 133.985) (end 156.845 139.065) (width 0.508) (layer B.Cu) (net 10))
 (segment (start 161.925 120.015) (end 161.925 133.985) (width 0.508) (layer B.Cu) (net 10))
 (segment (start 167.005 114.935) (end 161.925 120.015) (width 0.508) (layer B.Cu) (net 10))
 (segment (start 190.5 126.365) (end 190.5 121.92) (width 0.508) (layer B.Cu) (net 11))
 (segment (start 107.95 132.08) (end 107.315 132.715) (width 0.508) (layer B.Cu) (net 12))
 (segment (start 107.95 137.16) (end 106.68 135.89) (width 0.508) (layer B.Cu) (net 12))
 (segment (start 106.045 129.54) (end 109.22 129.54) (width 0.508) (layer B.Cu) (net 12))
 (segment (start 106.68 135.89) (end 106.045 135.255) (width 0.508) (layer B.Cu) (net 12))
 (segment (start 109.22 130.81) (end 109.22 129.54) (width 0.508) (layer B.Cu) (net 12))
 (segment (start 106.045 133.985) (end 107.315 132.715) (width 0.508) (layer B.Cu) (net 12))
 (segment (start 107.315 132.715) (end 109.22 130.81) (width 0.508) (layer B.Cu) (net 12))
 (segment (start 106.045 135.255) (end 106.045 133.985) (width 0.508) (layer B.Cu) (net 12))
 (segment (start 111.125 143.51) (end 104.14 136.525) (width 0.508) (layer B.Cu) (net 13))
 (segment (start 104.14 124.46) (end 109.22 119.38) (width 0.508) (layer B.Cu) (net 13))
 (segment (start 104.14 136.525) (end 104.14 124.46) (width 0.508) (layer B.Cu) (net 13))
 (segment (start 120.015 117.475) (end 114.3 117.475) (width 0.508) (layer B.Cu) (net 13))
 (segment (start 114.3 117.475) (end 112.395 119.38) (width 0.508) (layer B.Cu) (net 13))
 (segment (start 109.22 119.38) (end 112.395 119.38) (width 0.508) (layer B.Cu) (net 13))
 (segment (start 112.395 129.54) (end 115.57 129.54) (width 0.508) (layer B.Cu) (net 14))
 (segment (start 115.57 129.54) (end 120.65 129.54) (width 0.508) (layer B.Cu) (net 14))
 (segment (start 120.65 129.54) (end 121.92 128.27) (width 0.508) (layer B.Cu) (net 14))
 (segment (start 121.92 128.27) (end 121.92 126.365) (width 0.508) (layer B.Cu) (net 14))
 (segment (start 115.57 119.38) (end 119.38 123.19) (width 0.508) (layer B.Cu) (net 15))
 (segment (start 119.38 123.19) (end 119.38 126.365) (width 0.508) (layer B.Cu) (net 15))
 (segment (start 138.43 129.54) (end 135.255 129.54) (width 0.508) (layer B.Cu) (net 16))
 (segment (start 135.255 129.54) (end 132.08 126.365) (width 0.508) (layer B.Cu) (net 16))
 (segment (start 129.54 123.19) (end 132.08 123.19) (width 0.508) (layer B.Cu) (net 16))
 (segment (start 132.08 123.19) (end 132.08 126.365) (width 0.508) (layer B.Cu) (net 16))
 (segment (start 142.24 137.16) (end 142.24 129.54) (width 0.508) (layer B.Cu) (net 17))
 (segment (start 142.24 129.54) (end 139.065 126.365) (width 0.508) (layer B.Cu) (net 17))
 (segment (start 134.62 126.365) (end 139.065 126.365) (width 0.508) (layer B.Cu) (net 17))
 (segment (start 139.065 126.365) (end 145.415 126.365) (width 0.508) (layer B.Cu) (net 17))
 (segment (start 145.415 126.365) (end 148.59 129.54) (width 0.508) (layer B.Cu) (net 17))
 (segment (start 124.46 143.51) (end 121.285 143.51) (width 0.508) (layer B.Cu) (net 18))
 (segment (start 124.46 143.51) (end 128.905 143.51) (width 0.508) (layer B.Cu) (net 18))
 (segment (start 132.08 140.335) (end 132.08 137.16) (width 0.508) (layer B.Cu) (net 18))
 (segment (start 128.905 143.51) (end 132.08 140.335) (width 0.508) (layer B.Cu) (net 18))
 (segment (start 132.08 137.16) (end 132.08 133.985) (width 0.508) (layer B.Cu) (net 18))
 (segment (start 134.62 133.985) (end 134.62 140.335) (width 0.508) (layer B.Cu) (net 19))
 (segment (start 134.62 140.335) (end 134.62 143.51) (width 0.508) (layer B.Cu) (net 19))
 (segment (start 124.46 140.335) (end 124.46 139.7) (width 0.508) (layer B.Cu) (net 20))
 (segment (start 124.46 139.7) (end 121.92 137.16) (width 0.508) (layer B.Cu) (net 20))
 (segment (start 121.92 137.16) (end 121.92 133.985) (width 0.508) (layer B.Cu) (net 20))
 (segment (start 165.735 104.775) (end 165.735 104.14) (width 1.27) (layer B.Cu) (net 21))
 (segment (start 165.735 104.14) (end 163.83 102.235) (width 1.27) (layer B.Cu) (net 21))
 (segment (start 163.83 102.235) (end 113.665 102.235) (width 1.27) (layer B.Cu) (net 21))
 (segment (start 113.665 102.235) (end 102.235 113.665) (width 1.27) (layer B.Cu) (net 21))
 (segment (start 102.235 113.665) (end 102.235 137.795) (width 1.27) (layer B.Cu) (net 21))
 (segment (start 102.235 137.795) (end 110.49 146.05) (width 1.27) (layer B.Cu) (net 21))
 (segment (start 110.49 146.05) (end 113.03 146.05) (width 1.27) (layer B.Cu) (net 21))
 (segment (start 113.03 146.05) (end 116.205 142.875) (width 1.27) (layer B.Cu) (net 21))
 (segment (start 116.205 142.875) (end 116.205 137.16) (width 1.27) (layer B.Cu) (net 21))
 (segment (start 111.76 137.16) (end 116.205 137.16) (width 1.27) (layer B.Cu) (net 21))
 (segment (start 116.205 137.16) (end 119.38 133.985) (width 1.27) (layer B.Cu) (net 21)))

